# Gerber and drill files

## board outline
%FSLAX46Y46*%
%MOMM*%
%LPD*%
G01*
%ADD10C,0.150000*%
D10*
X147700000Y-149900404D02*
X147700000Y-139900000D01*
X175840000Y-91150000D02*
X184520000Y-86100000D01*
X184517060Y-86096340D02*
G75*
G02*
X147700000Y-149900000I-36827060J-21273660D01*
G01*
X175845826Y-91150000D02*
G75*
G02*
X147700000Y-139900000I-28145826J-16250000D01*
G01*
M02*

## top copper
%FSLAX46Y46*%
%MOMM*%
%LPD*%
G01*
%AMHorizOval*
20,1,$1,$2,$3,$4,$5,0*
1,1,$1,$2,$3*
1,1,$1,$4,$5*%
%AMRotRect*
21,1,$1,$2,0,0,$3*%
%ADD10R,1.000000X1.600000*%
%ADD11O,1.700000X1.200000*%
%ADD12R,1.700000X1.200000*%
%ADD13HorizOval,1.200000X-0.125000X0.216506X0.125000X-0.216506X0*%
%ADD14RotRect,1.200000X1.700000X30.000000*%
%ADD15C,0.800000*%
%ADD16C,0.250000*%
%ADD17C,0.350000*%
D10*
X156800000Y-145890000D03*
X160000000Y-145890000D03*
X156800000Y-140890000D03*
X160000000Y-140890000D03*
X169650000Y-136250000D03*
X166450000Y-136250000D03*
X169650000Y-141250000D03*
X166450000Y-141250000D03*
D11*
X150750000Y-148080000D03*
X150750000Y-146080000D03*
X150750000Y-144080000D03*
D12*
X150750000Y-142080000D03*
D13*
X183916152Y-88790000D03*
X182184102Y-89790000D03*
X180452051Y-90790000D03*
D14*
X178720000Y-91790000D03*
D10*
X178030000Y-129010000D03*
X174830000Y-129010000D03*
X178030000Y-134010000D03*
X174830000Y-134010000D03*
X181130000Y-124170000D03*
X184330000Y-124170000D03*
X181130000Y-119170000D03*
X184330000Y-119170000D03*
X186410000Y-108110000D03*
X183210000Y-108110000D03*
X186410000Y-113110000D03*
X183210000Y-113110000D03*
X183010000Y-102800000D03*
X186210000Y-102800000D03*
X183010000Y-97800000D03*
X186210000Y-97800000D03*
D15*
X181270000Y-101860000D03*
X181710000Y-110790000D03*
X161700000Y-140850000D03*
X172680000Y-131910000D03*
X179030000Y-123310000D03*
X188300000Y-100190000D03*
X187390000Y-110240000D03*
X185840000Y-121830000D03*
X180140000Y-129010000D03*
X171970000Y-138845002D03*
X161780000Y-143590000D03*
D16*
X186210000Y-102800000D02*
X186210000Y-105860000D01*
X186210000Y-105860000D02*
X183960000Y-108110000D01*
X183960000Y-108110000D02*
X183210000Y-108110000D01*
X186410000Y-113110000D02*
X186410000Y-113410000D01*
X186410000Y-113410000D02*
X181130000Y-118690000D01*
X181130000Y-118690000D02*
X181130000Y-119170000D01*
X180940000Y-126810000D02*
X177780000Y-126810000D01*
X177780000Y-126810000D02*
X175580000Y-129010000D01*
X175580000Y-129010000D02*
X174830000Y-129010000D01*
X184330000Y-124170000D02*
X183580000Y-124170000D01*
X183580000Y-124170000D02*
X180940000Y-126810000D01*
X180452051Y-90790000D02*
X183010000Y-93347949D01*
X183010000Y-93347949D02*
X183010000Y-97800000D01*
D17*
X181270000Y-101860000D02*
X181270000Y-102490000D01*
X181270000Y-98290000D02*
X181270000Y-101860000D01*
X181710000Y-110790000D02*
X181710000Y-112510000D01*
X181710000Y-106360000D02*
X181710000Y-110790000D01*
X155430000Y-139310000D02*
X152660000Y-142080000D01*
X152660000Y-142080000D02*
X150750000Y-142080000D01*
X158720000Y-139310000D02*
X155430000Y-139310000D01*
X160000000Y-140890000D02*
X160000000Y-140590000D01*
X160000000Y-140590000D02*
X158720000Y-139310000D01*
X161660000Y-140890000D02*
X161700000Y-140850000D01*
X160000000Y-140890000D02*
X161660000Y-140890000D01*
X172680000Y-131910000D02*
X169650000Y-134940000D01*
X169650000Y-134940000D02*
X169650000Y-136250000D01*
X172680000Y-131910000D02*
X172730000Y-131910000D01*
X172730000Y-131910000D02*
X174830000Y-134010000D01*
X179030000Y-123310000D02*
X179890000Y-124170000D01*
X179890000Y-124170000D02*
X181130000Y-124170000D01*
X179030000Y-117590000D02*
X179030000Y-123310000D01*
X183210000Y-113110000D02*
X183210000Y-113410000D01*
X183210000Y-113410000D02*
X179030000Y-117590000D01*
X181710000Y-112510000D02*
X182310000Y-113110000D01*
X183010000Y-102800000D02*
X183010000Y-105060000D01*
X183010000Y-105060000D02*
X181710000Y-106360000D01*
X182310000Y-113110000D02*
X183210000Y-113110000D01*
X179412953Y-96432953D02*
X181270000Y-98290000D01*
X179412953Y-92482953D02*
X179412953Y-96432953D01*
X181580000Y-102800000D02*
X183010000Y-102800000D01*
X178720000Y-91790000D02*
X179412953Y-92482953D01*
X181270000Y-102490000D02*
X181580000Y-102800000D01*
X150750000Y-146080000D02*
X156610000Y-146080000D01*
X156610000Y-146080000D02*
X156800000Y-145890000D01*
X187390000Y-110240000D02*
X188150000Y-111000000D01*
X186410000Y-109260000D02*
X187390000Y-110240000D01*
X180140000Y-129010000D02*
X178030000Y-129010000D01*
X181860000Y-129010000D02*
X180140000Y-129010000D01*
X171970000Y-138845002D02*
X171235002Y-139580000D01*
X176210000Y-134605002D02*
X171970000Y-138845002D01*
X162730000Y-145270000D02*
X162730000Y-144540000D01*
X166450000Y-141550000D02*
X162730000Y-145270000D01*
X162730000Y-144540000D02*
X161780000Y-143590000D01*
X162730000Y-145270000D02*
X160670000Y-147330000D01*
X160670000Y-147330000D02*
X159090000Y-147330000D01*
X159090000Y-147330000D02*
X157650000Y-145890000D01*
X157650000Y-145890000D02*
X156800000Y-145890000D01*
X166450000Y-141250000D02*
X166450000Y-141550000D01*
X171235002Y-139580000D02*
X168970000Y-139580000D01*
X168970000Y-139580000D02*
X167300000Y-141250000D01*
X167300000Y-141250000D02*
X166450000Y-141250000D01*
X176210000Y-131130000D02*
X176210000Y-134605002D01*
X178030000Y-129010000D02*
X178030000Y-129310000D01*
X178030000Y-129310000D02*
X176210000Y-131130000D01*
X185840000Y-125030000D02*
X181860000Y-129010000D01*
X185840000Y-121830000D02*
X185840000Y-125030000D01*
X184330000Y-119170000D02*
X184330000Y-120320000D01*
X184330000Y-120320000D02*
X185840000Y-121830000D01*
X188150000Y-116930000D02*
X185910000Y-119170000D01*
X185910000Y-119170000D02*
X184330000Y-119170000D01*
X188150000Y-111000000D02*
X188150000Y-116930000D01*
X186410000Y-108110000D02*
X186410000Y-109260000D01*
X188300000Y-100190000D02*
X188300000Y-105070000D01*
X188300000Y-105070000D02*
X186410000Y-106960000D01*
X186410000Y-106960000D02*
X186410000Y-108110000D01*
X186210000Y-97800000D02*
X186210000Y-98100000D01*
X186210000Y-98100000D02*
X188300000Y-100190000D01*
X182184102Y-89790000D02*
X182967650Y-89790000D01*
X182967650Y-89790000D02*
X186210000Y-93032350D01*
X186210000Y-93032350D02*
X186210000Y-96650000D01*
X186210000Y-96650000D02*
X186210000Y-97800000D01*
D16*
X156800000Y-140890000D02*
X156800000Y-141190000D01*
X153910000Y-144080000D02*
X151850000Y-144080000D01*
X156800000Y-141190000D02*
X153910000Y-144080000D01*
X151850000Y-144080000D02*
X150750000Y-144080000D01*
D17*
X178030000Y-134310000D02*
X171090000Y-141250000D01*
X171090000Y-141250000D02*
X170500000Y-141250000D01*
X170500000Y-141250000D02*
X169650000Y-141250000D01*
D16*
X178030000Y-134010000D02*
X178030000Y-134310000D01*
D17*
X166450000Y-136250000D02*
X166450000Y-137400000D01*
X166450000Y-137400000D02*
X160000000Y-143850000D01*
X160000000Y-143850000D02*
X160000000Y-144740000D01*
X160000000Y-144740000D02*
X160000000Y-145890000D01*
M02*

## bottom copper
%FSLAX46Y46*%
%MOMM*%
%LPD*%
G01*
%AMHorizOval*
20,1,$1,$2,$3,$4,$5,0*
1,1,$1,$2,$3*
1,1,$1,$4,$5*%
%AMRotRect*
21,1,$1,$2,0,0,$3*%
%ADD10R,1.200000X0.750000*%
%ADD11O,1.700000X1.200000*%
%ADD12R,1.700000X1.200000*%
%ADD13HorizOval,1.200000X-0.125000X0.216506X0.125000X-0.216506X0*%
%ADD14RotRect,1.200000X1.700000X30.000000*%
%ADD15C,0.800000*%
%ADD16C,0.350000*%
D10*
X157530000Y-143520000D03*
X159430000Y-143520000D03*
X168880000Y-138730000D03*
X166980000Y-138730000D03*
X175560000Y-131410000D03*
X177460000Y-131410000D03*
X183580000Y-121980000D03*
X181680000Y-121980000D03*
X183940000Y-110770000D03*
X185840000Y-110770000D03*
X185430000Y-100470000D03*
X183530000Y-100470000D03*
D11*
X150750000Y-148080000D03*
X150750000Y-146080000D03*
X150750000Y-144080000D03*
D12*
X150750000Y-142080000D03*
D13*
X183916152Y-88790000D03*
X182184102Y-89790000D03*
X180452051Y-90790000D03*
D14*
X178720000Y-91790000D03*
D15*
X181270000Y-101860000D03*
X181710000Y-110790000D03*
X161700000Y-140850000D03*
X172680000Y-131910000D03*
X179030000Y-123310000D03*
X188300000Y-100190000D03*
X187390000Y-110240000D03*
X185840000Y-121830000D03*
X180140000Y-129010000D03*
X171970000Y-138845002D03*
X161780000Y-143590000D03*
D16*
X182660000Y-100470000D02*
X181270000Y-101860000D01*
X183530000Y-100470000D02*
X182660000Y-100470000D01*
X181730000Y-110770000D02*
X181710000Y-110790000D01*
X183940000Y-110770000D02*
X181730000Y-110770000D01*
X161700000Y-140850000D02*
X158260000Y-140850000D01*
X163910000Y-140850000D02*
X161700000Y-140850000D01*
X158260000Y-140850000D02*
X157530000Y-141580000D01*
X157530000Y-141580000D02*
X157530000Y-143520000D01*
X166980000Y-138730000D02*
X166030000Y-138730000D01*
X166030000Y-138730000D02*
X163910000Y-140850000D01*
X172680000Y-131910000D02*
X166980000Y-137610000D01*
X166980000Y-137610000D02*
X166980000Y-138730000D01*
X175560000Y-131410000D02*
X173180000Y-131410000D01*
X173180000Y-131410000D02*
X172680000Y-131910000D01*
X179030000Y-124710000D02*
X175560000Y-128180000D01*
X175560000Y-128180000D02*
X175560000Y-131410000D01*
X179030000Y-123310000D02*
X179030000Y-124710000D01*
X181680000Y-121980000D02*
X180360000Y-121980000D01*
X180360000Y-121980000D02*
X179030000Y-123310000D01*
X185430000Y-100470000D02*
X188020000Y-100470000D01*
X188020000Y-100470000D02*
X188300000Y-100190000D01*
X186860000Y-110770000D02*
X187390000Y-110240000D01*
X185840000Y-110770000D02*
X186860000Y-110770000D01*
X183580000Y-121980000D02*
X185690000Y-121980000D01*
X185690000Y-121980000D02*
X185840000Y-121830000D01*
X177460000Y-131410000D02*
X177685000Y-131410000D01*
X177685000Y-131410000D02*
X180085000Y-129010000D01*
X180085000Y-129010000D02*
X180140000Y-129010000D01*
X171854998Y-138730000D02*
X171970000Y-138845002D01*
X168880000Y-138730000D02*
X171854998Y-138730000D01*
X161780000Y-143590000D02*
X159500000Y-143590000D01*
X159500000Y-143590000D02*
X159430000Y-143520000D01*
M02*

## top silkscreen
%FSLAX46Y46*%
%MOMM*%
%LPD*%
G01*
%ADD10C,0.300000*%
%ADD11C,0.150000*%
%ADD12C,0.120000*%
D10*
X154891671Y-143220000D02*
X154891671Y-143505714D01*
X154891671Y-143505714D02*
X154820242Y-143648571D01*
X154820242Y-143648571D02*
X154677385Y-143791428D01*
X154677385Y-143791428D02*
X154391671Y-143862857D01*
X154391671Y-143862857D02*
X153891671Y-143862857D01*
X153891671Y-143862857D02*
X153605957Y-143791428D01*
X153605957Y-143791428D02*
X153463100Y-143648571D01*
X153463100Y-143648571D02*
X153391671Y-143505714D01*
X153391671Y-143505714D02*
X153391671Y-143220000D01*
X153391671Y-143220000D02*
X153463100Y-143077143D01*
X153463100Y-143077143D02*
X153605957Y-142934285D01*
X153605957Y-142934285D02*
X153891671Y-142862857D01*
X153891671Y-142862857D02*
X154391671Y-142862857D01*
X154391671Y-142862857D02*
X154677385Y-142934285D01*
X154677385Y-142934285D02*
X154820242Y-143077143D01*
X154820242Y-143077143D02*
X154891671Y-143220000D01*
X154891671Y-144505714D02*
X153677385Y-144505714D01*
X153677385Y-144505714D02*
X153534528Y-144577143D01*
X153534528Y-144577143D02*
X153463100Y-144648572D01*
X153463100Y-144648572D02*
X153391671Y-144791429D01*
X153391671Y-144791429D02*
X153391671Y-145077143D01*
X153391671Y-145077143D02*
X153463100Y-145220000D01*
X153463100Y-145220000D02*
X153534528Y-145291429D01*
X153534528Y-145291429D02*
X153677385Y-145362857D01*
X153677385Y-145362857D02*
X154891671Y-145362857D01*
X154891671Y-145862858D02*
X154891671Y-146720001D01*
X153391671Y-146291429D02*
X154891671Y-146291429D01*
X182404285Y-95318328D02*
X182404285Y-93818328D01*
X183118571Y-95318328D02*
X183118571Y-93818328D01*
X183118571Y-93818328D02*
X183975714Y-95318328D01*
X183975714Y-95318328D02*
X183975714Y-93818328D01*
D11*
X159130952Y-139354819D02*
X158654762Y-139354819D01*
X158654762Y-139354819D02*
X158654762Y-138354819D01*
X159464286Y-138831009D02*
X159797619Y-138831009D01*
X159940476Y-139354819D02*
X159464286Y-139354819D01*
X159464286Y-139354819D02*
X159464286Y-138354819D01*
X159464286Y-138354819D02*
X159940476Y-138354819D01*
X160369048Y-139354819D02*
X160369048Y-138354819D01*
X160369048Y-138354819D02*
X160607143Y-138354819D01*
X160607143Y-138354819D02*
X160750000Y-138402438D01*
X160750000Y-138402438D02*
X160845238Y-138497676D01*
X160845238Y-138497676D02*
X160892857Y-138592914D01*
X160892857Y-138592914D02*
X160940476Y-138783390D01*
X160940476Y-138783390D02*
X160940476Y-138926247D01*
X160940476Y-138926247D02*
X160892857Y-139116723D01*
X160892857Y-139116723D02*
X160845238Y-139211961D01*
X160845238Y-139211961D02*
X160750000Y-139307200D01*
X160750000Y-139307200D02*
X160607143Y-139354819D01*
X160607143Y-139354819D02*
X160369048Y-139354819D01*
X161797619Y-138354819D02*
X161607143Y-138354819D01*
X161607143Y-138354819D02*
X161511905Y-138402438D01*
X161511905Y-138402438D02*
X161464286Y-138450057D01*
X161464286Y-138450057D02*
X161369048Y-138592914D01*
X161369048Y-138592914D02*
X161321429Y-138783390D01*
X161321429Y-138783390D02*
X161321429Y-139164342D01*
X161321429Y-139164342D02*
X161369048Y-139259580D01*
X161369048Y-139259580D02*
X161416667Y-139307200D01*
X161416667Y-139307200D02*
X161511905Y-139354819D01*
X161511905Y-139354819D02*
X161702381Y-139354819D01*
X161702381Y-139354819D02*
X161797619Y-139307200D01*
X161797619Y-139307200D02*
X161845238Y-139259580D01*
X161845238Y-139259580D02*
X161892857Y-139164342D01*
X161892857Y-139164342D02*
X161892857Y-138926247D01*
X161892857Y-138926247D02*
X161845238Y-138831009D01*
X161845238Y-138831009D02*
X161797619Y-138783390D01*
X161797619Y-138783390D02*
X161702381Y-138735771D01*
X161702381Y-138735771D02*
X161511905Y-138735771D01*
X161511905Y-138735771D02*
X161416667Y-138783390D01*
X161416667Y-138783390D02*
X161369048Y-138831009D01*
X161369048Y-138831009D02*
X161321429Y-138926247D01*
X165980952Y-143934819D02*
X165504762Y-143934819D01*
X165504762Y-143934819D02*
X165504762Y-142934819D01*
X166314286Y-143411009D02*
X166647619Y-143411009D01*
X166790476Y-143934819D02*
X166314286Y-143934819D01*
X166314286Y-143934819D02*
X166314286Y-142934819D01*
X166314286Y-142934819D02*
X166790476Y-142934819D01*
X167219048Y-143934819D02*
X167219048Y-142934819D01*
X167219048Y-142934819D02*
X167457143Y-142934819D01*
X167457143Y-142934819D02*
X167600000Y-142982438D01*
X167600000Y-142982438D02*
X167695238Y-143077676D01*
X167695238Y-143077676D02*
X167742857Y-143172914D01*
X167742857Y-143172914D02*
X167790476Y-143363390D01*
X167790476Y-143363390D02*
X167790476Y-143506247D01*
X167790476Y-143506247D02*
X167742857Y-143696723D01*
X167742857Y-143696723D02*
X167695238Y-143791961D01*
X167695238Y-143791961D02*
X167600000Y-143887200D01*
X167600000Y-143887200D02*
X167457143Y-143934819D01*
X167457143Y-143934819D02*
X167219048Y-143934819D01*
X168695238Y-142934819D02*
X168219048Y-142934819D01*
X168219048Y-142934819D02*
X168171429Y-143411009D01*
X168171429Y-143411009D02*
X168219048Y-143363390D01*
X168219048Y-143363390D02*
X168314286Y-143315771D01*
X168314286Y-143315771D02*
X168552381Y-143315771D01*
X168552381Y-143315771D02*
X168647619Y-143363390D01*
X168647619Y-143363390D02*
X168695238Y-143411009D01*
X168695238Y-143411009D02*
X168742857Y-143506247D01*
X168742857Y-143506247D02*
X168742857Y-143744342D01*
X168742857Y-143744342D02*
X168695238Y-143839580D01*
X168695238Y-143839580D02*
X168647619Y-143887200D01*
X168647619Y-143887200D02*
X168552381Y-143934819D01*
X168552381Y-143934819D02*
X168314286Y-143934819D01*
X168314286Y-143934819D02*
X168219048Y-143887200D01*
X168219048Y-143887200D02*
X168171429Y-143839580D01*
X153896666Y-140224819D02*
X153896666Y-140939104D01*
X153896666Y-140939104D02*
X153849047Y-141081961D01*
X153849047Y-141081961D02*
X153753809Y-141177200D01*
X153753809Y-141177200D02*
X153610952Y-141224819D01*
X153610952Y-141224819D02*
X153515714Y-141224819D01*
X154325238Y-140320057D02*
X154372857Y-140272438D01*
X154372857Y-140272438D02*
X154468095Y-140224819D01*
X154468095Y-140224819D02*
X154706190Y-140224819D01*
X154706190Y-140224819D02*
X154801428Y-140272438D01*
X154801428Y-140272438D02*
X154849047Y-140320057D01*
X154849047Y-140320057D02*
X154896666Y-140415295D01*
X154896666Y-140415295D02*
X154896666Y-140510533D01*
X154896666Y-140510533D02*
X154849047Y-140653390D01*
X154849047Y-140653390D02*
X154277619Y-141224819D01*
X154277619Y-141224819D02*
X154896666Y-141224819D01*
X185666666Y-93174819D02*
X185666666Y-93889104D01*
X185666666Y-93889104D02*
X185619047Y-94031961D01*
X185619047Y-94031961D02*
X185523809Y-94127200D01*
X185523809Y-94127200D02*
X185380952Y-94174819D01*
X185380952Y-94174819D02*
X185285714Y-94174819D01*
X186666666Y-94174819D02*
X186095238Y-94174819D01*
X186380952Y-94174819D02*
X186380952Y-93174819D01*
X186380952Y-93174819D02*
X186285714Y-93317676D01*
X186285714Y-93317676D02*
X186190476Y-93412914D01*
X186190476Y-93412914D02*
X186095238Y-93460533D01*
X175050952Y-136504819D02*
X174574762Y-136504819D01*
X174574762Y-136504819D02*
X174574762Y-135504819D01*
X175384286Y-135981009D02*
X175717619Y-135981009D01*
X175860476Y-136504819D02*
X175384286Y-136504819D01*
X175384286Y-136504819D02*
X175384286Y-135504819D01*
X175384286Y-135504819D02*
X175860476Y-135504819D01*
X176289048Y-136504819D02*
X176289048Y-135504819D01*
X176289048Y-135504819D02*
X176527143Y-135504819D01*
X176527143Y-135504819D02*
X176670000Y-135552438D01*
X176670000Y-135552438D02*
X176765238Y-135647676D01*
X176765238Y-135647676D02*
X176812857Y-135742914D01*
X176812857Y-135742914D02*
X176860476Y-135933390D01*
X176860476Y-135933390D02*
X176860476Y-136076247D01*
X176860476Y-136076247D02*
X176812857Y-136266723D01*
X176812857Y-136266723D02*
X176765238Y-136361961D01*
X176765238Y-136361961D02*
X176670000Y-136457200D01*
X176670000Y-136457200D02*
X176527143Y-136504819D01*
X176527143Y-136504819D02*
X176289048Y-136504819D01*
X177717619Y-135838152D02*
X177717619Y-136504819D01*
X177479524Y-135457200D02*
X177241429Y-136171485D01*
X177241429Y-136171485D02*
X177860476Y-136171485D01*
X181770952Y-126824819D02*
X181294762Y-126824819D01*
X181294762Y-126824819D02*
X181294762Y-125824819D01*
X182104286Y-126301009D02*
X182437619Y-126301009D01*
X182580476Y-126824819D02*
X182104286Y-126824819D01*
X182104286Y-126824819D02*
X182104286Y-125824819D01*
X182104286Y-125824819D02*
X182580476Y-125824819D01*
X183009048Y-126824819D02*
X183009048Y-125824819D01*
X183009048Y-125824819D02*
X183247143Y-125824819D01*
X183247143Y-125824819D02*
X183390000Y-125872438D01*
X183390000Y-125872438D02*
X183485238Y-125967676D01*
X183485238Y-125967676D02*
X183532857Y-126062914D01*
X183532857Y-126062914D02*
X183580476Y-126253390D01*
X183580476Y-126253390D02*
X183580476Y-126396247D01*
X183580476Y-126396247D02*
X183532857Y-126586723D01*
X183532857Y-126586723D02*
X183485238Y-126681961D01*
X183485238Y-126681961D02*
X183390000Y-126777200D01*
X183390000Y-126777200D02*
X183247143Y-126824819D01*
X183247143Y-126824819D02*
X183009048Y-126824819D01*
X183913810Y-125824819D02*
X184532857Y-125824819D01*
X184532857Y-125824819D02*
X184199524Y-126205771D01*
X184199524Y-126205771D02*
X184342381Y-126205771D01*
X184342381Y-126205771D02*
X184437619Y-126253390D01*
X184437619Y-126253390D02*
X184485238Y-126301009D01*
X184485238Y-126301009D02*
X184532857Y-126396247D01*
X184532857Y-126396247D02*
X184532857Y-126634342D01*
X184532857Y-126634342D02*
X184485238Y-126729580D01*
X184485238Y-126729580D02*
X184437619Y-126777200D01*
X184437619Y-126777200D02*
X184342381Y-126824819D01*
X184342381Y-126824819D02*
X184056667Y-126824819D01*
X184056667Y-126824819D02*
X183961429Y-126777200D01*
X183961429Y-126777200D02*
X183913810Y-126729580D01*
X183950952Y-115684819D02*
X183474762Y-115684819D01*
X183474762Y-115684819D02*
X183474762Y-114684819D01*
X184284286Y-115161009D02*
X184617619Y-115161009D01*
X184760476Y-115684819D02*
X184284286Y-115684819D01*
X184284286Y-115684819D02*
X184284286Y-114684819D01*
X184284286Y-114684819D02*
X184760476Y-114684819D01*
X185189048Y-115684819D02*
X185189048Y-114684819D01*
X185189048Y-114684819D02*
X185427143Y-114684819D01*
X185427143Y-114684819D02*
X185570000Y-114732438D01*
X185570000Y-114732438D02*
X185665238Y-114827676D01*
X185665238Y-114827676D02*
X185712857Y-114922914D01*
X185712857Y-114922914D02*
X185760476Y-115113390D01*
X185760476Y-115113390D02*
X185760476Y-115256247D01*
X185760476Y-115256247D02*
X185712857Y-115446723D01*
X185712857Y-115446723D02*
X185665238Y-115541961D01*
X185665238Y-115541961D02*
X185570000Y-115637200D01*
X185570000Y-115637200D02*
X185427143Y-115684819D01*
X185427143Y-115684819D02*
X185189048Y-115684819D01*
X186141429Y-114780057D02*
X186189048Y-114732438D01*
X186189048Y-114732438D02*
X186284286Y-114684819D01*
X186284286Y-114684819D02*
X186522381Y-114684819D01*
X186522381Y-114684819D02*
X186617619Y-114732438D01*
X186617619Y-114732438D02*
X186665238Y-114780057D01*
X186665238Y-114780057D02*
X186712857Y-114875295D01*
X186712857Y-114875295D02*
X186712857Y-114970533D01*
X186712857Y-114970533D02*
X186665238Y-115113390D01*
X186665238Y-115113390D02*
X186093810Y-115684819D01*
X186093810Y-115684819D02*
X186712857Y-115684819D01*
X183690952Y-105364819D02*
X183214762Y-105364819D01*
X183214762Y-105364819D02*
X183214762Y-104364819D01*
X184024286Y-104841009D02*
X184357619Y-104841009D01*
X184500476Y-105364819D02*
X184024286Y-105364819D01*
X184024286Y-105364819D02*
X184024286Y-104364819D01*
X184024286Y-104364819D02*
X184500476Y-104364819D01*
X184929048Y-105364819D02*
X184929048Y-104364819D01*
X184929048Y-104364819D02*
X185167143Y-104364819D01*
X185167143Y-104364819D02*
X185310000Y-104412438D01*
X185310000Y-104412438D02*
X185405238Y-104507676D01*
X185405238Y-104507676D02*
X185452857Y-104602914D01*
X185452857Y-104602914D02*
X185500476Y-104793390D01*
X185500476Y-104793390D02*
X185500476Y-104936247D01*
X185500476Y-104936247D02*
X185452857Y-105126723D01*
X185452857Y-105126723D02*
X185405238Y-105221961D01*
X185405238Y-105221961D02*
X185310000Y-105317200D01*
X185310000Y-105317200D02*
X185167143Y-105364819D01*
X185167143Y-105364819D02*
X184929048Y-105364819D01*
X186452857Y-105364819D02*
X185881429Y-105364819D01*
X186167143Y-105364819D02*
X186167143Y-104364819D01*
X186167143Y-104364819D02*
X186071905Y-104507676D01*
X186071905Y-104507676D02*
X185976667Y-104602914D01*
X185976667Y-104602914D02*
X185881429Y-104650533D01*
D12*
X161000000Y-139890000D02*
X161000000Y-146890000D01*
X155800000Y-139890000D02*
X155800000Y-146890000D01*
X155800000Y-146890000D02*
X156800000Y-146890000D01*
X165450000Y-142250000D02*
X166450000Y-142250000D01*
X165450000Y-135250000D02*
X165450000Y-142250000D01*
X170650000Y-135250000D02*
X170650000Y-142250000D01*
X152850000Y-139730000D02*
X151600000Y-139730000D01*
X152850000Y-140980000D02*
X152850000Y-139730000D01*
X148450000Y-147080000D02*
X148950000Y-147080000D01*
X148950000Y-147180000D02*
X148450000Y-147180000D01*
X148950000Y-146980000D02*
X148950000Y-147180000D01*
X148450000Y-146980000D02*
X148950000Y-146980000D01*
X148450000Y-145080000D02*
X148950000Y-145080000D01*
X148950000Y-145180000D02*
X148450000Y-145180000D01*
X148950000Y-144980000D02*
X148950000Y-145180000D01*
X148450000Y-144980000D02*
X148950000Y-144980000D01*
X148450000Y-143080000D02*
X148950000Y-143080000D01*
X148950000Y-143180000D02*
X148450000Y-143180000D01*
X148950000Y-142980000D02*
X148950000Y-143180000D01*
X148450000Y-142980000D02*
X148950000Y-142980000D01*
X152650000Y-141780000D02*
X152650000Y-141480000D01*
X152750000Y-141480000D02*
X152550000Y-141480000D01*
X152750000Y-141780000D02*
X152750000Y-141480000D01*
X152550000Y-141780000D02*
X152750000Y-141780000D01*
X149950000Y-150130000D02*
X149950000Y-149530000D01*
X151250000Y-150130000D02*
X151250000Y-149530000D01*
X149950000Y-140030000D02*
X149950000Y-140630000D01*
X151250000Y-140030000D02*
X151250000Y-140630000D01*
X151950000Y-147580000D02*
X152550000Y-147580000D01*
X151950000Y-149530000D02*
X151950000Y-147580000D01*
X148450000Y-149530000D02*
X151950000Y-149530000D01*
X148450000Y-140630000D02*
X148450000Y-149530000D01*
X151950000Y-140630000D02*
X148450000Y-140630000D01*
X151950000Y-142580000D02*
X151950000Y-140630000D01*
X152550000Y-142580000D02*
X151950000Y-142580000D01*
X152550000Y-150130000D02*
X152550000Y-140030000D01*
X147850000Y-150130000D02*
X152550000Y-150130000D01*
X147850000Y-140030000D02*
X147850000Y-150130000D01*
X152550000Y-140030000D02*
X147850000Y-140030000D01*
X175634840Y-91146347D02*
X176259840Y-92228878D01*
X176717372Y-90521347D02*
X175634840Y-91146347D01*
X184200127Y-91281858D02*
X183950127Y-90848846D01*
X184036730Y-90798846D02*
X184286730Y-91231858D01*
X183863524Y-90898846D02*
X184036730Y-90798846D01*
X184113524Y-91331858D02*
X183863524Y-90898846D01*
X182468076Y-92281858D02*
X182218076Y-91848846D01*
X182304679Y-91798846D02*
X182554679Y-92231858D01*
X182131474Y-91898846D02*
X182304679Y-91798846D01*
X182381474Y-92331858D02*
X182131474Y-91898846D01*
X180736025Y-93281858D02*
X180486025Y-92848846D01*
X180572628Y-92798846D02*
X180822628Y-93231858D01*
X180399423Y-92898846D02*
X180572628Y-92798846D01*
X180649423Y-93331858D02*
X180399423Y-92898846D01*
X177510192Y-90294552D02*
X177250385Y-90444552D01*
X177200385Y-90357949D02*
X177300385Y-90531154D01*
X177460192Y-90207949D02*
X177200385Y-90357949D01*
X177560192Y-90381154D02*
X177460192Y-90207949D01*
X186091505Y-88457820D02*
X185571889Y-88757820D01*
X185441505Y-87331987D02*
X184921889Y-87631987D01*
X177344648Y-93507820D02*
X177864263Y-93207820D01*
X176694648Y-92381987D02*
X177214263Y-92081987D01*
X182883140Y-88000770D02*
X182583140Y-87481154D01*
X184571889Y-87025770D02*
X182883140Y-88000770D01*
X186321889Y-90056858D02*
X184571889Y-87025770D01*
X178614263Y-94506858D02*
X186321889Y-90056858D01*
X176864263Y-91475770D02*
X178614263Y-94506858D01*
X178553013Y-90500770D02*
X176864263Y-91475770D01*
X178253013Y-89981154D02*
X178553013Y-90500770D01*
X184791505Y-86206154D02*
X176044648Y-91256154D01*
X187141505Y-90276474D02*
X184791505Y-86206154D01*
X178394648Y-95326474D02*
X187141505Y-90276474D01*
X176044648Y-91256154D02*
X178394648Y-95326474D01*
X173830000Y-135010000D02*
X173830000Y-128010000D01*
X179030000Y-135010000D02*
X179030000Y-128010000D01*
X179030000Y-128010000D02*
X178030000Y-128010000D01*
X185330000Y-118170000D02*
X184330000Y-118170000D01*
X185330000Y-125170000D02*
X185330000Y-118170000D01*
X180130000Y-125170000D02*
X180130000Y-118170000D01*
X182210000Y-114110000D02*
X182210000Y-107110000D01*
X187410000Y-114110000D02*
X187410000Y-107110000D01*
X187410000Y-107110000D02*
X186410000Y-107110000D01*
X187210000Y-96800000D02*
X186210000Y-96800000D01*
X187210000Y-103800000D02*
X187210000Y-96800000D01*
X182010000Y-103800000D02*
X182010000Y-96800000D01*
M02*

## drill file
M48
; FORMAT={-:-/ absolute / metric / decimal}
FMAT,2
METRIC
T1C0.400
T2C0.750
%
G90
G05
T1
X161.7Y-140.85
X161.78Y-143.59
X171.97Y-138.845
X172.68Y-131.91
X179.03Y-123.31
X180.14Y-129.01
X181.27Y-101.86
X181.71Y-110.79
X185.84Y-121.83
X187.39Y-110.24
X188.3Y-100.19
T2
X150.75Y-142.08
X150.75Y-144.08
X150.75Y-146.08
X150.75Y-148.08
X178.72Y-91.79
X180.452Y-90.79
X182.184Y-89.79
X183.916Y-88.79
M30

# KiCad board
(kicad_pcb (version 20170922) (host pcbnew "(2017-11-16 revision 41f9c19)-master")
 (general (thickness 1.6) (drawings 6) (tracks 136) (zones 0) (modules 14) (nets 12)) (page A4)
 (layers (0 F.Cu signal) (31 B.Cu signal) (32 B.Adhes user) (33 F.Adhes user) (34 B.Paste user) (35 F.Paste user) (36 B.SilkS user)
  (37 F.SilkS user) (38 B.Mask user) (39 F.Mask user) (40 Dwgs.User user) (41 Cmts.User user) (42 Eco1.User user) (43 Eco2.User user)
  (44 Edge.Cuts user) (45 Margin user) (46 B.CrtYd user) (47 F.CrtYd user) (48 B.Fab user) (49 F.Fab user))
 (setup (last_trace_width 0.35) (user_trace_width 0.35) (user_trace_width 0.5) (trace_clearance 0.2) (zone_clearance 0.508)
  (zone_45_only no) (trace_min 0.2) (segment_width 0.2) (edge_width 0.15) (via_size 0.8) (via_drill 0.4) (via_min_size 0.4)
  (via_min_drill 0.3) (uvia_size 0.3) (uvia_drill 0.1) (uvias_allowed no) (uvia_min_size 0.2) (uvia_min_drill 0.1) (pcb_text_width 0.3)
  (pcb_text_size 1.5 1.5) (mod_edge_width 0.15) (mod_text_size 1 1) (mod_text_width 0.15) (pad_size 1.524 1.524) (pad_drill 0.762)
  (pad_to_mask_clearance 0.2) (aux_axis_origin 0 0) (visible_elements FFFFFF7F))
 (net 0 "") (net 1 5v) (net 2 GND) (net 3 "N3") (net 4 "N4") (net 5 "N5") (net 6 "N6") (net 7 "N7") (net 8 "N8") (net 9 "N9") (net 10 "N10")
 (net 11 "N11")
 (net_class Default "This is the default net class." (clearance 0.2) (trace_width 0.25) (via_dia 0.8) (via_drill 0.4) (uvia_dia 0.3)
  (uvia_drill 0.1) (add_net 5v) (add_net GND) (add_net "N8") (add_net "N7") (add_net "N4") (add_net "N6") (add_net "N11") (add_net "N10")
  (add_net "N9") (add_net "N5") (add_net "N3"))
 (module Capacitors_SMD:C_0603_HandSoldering (layer B.Cu) (at 158.48 143.52)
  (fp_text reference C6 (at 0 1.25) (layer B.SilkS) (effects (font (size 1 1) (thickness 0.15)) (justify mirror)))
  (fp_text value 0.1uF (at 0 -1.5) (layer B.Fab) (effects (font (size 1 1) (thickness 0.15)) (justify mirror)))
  (pad 1 smd rect (at -0.95 0) (size 1.2 0.75) (layers B.Cu B.Paste B.Mask) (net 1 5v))
  (pad 2 smd rect (at 0.95 0) (size 1.2 0.75) (layers B.Cu B.Paste B.Mask) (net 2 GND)))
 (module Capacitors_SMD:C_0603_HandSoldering (layer B.Cu) (at 167.93 138.73)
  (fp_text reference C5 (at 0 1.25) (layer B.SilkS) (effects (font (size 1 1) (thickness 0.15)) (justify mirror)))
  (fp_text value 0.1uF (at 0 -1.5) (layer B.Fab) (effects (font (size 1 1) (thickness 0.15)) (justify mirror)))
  (pad 2 smd rect (at 0.95 0) (size 1.2 0.75) (layers B.Cu B.Paste B.Mask) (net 2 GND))
  (pad 1 smd rect (at -0.95 0) (size 1.2 0.75) (layers B.Cu B.Paste B.Mask) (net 1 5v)))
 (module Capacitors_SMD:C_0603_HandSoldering (layer B.Cu) (at 176.51 131.41)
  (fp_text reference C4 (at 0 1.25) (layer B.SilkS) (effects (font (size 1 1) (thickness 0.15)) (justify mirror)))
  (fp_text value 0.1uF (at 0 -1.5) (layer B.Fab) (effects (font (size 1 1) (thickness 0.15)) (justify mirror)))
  (pad 1 smd rect (at -0.95 0) (size 1.2 0.75) (layers B.Cu B.Paste B.Mask) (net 1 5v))
  (pad 2 smd rect (at 0.95 0) (size 1.2 0.75) (layers B.Cu B.Paste B.Mask) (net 2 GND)))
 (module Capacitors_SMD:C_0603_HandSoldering (layer B.Cu) (at 182.63 121.98)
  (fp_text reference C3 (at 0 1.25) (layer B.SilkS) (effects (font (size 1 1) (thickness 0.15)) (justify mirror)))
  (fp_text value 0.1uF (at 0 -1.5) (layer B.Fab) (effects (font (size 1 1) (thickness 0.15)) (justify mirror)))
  (pad 2 smd rect (at 0.95 0) (size 1.2 0.75) (layers B.Cu B.Paste B.Mask) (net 2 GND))
  (pad 1 smd rect (at -0.95 0) (size 1.2 0.75) (layers B.Cu B.Paste B.Mask) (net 1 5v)))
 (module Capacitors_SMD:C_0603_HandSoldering (layer B.Cu) (at 184.89 110.77)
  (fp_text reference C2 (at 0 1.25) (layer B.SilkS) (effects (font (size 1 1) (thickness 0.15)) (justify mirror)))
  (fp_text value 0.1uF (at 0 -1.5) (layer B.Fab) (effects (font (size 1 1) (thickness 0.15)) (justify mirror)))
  (pad 1 smd rect (at -0.95 0) (size 1.2 0.75) (layers B.Cu B.Paste B.Mask) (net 1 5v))
  (pad 2 smd rect (at 0.95 0) (size 1.2 0.75) (layers B.Cu B.Paste B.Mask) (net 2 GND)))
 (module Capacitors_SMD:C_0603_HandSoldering (layer B.Cu) (at 184.48 100.47)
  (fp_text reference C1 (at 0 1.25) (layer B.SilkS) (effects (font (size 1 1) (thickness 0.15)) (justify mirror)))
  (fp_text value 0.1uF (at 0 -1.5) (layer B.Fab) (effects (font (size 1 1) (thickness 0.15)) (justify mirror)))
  (pad 2 smd rect (at 0.95 0) (size 1.2 0.75) (layers B.Cu B.Paste B.Mask) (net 2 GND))
  (pad 1 smd rect (at -0.95 0) (size 1.2 0.75) (layers B.Cu B.Paste B.Mask) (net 1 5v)))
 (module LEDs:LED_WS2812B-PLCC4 (layer F.Cu) (at 158.4 143.39 270)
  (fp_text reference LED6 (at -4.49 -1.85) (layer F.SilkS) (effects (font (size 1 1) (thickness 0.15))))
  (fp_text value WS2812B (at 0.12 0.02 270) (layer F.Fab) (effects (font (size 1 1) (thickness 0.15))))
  (fp_line (start -3.5 -2.6) (end 3.5 -2.6) (layer F.SilkS) (width 0.12))
  (fp_line (start -3.5 2.6) (end 3.5 2.6) (layer F.SilkS) (width 0.12))
  (fp_line (start 3.5 2.6) (end 3.5 1.6) (layer F.SilkS) (width 0.12))
  (pad 3 smd rect (at 2.5 1.6 270) (size 1.6 1) (layers F.Cu F.Paste F.Mask) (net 2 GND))
  (pad 4 smd rect (at 2.5 -1.6 270) (size 1.6 1) (layers F.Cu F.Paste F.Mask) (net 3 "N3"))
  (pad 2 smd rect (at -2.5 1.6 270) (size 1.6 1) (layers F.Cu F.Paste F.Mask) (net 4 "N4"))
  (pad 1 smd rect (at -2.5 -1.6 270) (size 1.6 1) (layers F.Cu F.Paste F.Mask) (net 1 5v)))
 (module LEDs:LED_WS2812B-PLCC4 (layer F.Cu) (at 168.05 138.75 270)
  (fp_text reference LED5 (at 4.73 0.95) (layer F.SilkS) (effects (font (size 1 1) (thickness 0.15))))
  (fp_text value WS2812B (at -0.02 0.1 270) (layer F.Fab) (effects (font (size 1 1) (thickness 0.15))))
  (fp_line (start 3.5 2.6) (end 3.5 1.6) (layer F.SilkS) (width 0.12))
  (fp_line (start -3.5 2.6) (end 3.5 2.6) (layer F.SilkS) (width 0.12))
  (fp_line (start -3.5 -2.6) (end 3.5 -2.6) (layer F.SilkS) (width 0.12))
  (pad 1 smd rect (at -2.5 -1.6 270) (size 1.6 1) (layers F.Cu F.Paste F.Mask) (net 1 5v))
  (pad 2 smd rect (at -2.5 1.6 270) (size 1.6 1) (layers F.Cu F.Paste F.Mask) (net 3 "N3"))
  (pad 4 smd rect (at 2.5 -1.6 270) (size 1.6 1) (layers F.Cu F.Paste F.Mask) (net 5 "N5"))
  (pad 3 smd rect (at 2.5 1.6 270) (size 1.6 1) (layers F.Cu F.Paste F.Mask) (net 2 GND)))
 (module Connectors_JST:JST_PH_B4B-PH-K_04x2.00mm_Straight (layer F.Cu) (at 150.75 142.08 270)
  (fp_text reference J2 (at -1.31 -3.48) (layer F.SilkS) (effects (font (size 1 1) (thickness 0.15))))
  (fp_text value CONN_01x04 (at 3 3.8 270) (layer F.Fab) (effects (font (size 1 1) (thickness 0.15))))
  (fp_line (start -2.35 -2.1) (end -2.35 -0.85) (layer F.SilkS) (width 0.12))
  (fp_line (start -1.1 -2.1) (end -2.35 -2.1) (layer F.SilkS) (width 0.12))
  (fp_line (start 5 2.3) (end 5 1.8) (layer F.SilkS) (width 0.12))
  (fp_line (start 5.1 1.8) (end 5.1 2.3) (layer F.SilkS) (width 0.12))
  (fp_line (start 4.9 1.8) (end 5.1 1.8) (layer F.SilkS) (width 0.12))
  (fp_line (start 4.9 2.3) (end 4.9 1.8) (layer F.SilkS) (width 0.12))
  (fp_line (start 3 2.3) (end 3 1.8) (layer F.SilkS) (width 0.12))
  (fp_line (start 3.1 1.8) (end 3.1 2.3) (layer F.SilkS) (width 0.12))
  (fp_line (start 2.9 1.8) (end 3.1 1.8) (layer F.SilkS) (width 0.12))
  (fp_line (start 2.9 2.3) (end 2.9 1.8) (layer F.SilkS) (width 0.12))
  (fp_line (start 1 2.3) (end 1 1.8) (layer F.SilkS) (width 0.12))
  (fp_line (start 1.1 1.8) (end 1.1 2.3) (layer F.SilkS) (width 0.12))
  (fp_line (start 0.9 1.8) (end 1.1 1.8) (layer F.SilkS) (width 0.12))
  (fp_line (start 0.9 2.3) (end 0.9 1.8) (layer F.SilkS) (width 0.12))
  (fp_line (start -0.3 -1.9) (end -0.6 -1.9) (layer F.SilkS) (width 0.12))
  (fp_line (start -0.6 -2) (end -0.6 -1.8) (layer F.SilkS) (width 0.12))
  (fp_line (start -0.3 -2) (end -0.6 -2) (layer F.SilkS) (width 0.12))
  (fp_line (start -0.3 -1.8) (end -0.3 -2) (layer F.SilkS) (width 0.12))
  (fp_line (start 8.05 0.8) (end 7.45 0.8) (layer F.SilkS) (width 0.12))
  (fp_line (start 8.05 -0.5) (end 7.45 -0.5) (layer F.SilkS) (width 0.12))
  (fp_line (start -2.05 0.8) (end -1.45 0.8) (layer F.SilkS) (width 0.12))
  (fp_line (start -2.05 -0.5) (end -1.45 -0.5) (layer F.SilkS) (width 0.12))
  (fp_line (start 5.5 -1.2) (end 5.5 -1.8) (layer F.SilkS) (width 0.12))
  (fp_line (start 7.45 -1.2) (end 5.5 -1.2) (layer F.SilkS) (width 0.12))
  (fp_line (start 7.45 2.3) (end 7.45 -1.2) (layer F.SilkS) (width 0.12))
  (fp_line (start -1.45 2.3) (end 7.45 2.3) (layer F.SilkS) (width 0.12))
  (fp_line (start -1.45 -1.2) (end -1.45 2.3) (layer F.SilkS) (width 0.12))
  (fp_line (start 0.5 -1.2) (end -1.45 -1.2) (layer F.SilkS) (width 0.12))
  (fp_line (start 0.5 -1.8) (end 0.5 -1.2) (layer F.SilkS) (width 0.12))
  (fp_line (start 8.05 -1.8) (end -2.05 -1.8) (layer F.SilkS) (width 0.12))
  (fp_line (start 8.05 2.9) (end 8.05 -1.8) (layer F.SilkS) (width 0.12))
  (fp_line (start -2.05 2.9) (end 8.05 2.9) (layer F.SilkS) (width 0.12))
  (fp_line (start -2.05 -1.8) (end -2.05 2.9) (layer F.SilkS) (width 0.12))
  (pad 4 thru_hole oval (at 6 0 270) (size 1.2 1.7) (drill 0.75) (layers *.Cu *.Mask) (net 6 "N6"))
  (pad 3 thru_hole oval (at 4 0 270) (size 1.2 1.7) (drill 0.75) (layers *.Cu *.Mask) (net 2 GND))
  (pad 2 thru_hole oval (at 2 0 270) (size 1.2 1.7) (drill 0.75) (layers *.Cu *.Mask) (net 4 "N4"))
  (pad 1 thru_hole rect (at 0 0 270) (size 1.2 1.7) (drill 0.75) (layers *.Cu *.Mask) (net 1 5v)))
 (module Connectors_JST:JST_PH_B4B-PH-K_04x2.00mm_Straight (layer F.Cu) (at 178.72 91.79 30)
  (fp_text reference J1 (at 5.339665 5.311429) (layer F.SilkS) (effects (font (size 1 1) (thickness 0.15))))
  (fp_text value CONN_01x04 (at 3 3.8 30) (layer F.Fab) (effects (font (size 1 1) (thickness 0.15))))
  (fp_line (start -2.35 -2.1) (end -2.35 -0.85) (layer F.SilkS) (width 0.12))
  (fp_line (start -1.1 -2.1) (end -2.35 -2.1) (layer F.SilkS) (width 0.12))
  (fp_line (start 5 2.3) (end 5 1.8) (layer F.SilkS) (width 0.12))
  (fp_line (start 5.1 1.8) (end 5.1 2.3) (layer F.SilkS) (width 0.12))
  (fp_line (start 4.9 1.8) (end 5.1 1.8) (layer F.SilkS) (width 0.12))
  (fp_line (start 4.9 2.3) (end 4.9 1.8) (layer F.SilkS) (width 0.12))
  (fp_line (start 3 2.3) (end 3 1.8) (layer F.SilkS) (width 0.12))
  (fp_line (start 3.1 1.8) (end 3.1 2.3) (layer F.SilkS) (width 0.12))
  (fp_line (start 2.9 1.8) (end 3.1 1.8) (layer F.SilkS) (width 0.12))
  (fp_line (start 2.9 2.3) (end 2.9 1.8) (layer F.SilkS) (width 0.12))
  (fp_line (start 1 2.3) (end 1 1.8) (layer F.SilkS) (width 0.12))
  (fp_line (start 1.1 1.8) (end 1.1 2.3) (layer F.SilkS) (width 0.12))
  (fp_line (start 0.9 1.8) (end 1.1 1.8) (layer F.SilkS) (width 0.12))
  (fp_line (start 0.9 2.3) (end 0.9 1.8) (layer F.SilkS) (width 0.12))
  (fp_line (start -0.3 -1.9) (end -0.6 -1.9) (layer F.SilkS) (width 0.12))
  (fp_line (start -0.6 -2) (end -0.6 -1.8) (layer F.SilkS) (width 0.12))
  (fp_line (start -0.3 -2) (end -0.6 -2) (layer F.SilkS) (width 0.12))
  (fp_line (start -0.3 -1.8) (end -0.3 -2) (layer F.SilkS) (width 0.12))
  (fp_line (start 8.05 0.8) (end 7.45 0.8) (layer F.SilkS) (width 0.12))
  (fp_line (start 8.05 -0.5) (end 7.45 -0.5) (layer F.SilkS) (width 0.12))
  (fp_line (start -2.05 0.8) (end -1.45 0.8) (layer F.SilkS) (width 0.12))
  (fp_line (start -2.05 -0.5) (end -1.45 -0.5) (layer F.SilkS) (width 0.12))
  (fp_line (start 5.5 -1.2) (end 5.5 -1.8) (layer F.SilkS) (width 0.12))
  (fp_line (start 7.45 -1.2) (end 5.5 -1.2) (layer F.SilkS) (width 0.12))
  (fp_line (start 7.45 2.3) (end 7.45 -1.2) (layer F.SilkS) (width 0.12))
  (fp_line (start -1.45 2.3) (end 7.45 2.3) (layer F.SilkS) (width 0.12))
  (fp_line (start -1.45 -1.2) (end -1.45 2.3) (layer F.SilkS) (width 0.12))
  (fp_line (start 0.5 -1.2) (end -1.45 -1.2) (layer F.SilkS) (width 0.12))
  (fp_line (start 0.5 -1.8) (end 0.5 -1.2) (layer F.SilkS) (width 0.12))
  (fp_line (start 8.05 -1.8) (end -2.05 -1.8) (layer F.SilkS) (width 0.12))
  (fp_line (start 8.05 2.9) (end 8.05 -1.8) (layer F.SilkS) (width 0.12))
  (fp_line (start -2.05 2.9) (end 8.05 2.9) (layer F.SilkS) (width 0.12))
  (fp_line (start -2.05 -1.8) (end -2.05 2.9) (layer F.SilkS) (width 0.12))
  (pad 4 thru_hole oval (at 6 0 30) (size 1.2 1.7) (drill 0.75) (layers *.Cu *.Mask) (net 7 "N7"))
  (pad 3 thru_hole oval (at 4 0 30) (size 1.2 1.7) (drill 0.75) (layers *.Cu *.Mask) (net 2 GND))
  (pad 2 thru_hole oval (at 2 0 30) (size 1.2 1.7) (drill 0.75) (layers *.Cu *.Mask) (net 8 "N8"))
  (pad 1 thru_hole rect (at 0 0 30) (size 1.2 1.7) (drill 0.75) (layers *.Cu *.Mask) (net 1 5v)))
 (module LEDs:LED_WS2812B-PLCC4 (layer F.Cu) (at 176.43 131.51 90)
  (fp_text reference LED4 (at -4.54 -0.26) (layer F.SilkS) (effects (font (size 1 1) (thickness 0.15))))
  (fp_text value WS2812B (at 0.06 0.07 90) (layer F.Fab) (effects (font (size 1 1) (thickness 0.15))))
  (fp_line (start -3.5 -2.6) (end 3.5 -2.6) (layer F.SilkS) (width 0.12))
  (fp_line (start -3.5 2.6) (end 3.5 2.6) (layer F.SilkS) (width 0.12))
  (fp_line (start 3.5 2.6) (end 3.5 1.6) (layer F.SilkS) (width 0.12))
  (pad 3 smd rect (at 2.5 1.6 90) (size 1.6 1) (layers F.Cu F.Paste F.Mask) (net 2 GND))
  (pad 4 smd rect (at 2.5 -1.6 90) (size 1.6 1) (layers F.Cu F.Paste F.Mask) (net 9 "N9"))
  (pad 2 smd rect (at -2.5 1.6 90) (size 1.6 1) (layers F.Cu F.Paste F.Mask) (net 5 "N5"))
  (pad 1 smd rect (at -2.5 -1.6 90) (size 1.6 1) (layers F.Cu F.Paste F.Mask) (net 1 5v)))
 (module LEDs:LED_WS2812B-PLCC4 (layer F.Cu) (at 182.73 121.67 90)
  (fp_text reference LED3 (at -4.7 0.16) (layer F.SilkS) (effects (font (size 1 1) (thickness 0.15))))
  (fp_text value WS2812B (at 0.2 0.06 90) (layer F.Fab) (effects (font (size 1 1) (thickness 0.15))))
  (fp_line (start 3.5 2.6) (end 3.5 1.6) (layer F.SilkS) (width 0.12))
  (fp_line (start -3.5 2.6) (end 3.5 2.6) (layer F.SilkS) (width 0.12))
  (fp_line (start -3.5 -2.6) (end 3.5 -2.6) (layer F.SilkS) (width 0.12))
  (pad 1 smd rect (at -2.5 -1.6 90) (size 1.6 1) (layers F.Cu F.Paste F.Mask) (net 1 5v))
  (pad 2 smd rect (at -2.5 1.6 90) (size 1.6 1) (layers F.Cu F.Paste F.Mask) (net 9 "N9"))
  (pad 4 smd rect (at 2.5 -1.6 90) (size 1.6 1) (layers F.Cu F.Paste F.Mask) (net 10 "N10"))
  (pad 3 smd rect (at 2.5 1.6 90) (size 1.6 1) (layers F.Cu F.Paste F.Mask) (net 2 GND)))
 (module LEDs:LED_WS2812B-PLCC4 (layer F.Cu) (at 184.81 110.61 90)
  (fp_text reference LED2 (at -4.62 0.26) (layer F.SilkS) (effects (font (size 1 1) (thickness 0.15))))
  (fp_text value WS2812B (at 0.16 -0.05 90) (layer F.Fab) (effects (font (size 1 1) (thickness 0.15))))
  (fp_line (start -3.5 -2.6) (end 3.5 -2.6) (layer F.SilkS) (width 0.12))
  (fp_line (start -3.5 2.6) (end 3.5 2.6) (layer F.SilkS) (width 0.12))
  (fp_line (start 3.5 2.6) (end 3.5 1.6) (layer F.SilkS) (width 0.12))
  (pad 3 smd rect (at 2.5 1.6 90) (size 1.6 1) (layers F.Cu F.Paste F.Mask) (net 2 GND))
  (pad 4 smd rect (at 2.5 -1.6 90) (size 1.6 1) (layers F.Cu F.Paste F.Mask) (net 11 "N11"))
  (pad 2 smd rect (at -2.5 1.6 90) (size 1.6 1) (layers F.Cu F.Paste F.Mask) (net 10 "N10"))
  (pad 1 smd rect (at -2.5 -1.6 90) (size 1.6 1) (layers F.Cu F.Paste F.Mask) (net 1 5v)))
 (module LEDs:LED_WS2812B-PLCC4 (layer F.Cu) (at 184.61 100.3 90)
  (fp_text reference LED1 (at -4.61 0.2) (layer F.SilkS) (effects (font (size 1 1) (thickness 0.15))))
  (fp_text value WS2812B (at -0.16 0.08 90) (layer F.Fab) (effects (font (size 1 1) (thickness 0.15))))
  (fp_line (start 3.5 2.6) (end 3.5 1.6) (layer F.SilkS) (width 0.12))
  (fp_line (start -3.5 2.6) (end 3.5 2.6) (layer F.SilkS) (width 0.12))
  (fp_line (start -3.5 -2.6) (end 3.5 -2.6) (layer F.SilkS) (width 0.12))
  (pad 1 smd rect (at -2.5 -1.6 90) (size 1.6 1) (layers F.Cu F.Paste F.Mask) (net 1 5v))
  (pad 2 smd rect (at -2.5 1.6 90) (size 1.6 1) (layers F.Cu F.Paste F.Mask) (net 11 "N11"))
  (pad 4 smd rect (at 2.5 -1.6 90) (size 1.6 1) (layers F.Cu F.Paste F.Mask) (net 8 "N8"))
  (pad 3 smd rect (at 2.5 1.6 90) (size 1.6 1) (layers F.Cu F.Paste F.Mask) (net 2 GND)))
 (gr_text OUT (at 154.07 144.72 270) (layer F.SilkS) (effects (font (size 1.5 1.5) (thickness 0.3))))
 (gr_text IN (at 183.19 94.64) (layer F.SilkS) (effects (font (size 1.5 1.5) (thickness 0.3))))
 (gr_line (start 147.7 149.900404) (end 147.7 139.9) (layer Edge.Cuts) (width 0.15))
 (gr_line (start 175.84 91.15) (end 184.52 86.1) (layer Edge.Cuts) (width 0.15))
 (gr_arc (start 147.69 107.37) (end 147.7 149.9) (angle -120) (layer Edge.Cuts) (width 0.15))
 (gr_arc (start 147.7 107.4) (end 147.7 139.9) (angle -120) (layer Edge.Cuts) (width 0.15))
 (segment (start 186.21 102.8) (end 186.21 105.86) (width 0.25) (layer F.Cu) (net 11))
 (segment (start 186.21 105.86) (end 183.96 108.11) (width 0.25) (layer F.Cu) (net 11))
 (segment (start 183.96 108.11) (end 183.21 108.11) (width 0.25) (layer F.Cu) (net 11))
 (segment (start 186.41 113.11) (end 186.41 113.41) (width 0.25) (layer F.Cu) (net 10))
 (segment (start 186.41 113.41) (end 181.13 118.69) (width 0.25) (layer F.Cu) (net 10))
 (segment (start 181.13 118.69) (end 181.13 119.17) (width 0.25) (layer F.Cu) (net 10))
 (segment (start 180.94 126.81) (end 177.78 126.81) (width 0.25) (layer F.Cu) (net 9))
 (segment (start 177.78 126.81) (end 175.58 129.01) (width 0.25) (layer F.Cu) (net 9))
 (segment (start 175.58 129.01) (end 174.83 129.01) (width 0.25) (layer F.Cu) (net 9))
 (segment (start 184.33 124.17) (end 183.58 124.17) (width 0.25) (layer F.Cu) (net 9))
 (segment (start 183.58 124.17) (end 180.94 126.81) (width 0.25) (layer F.Cu) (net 9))
 (segment (start 180.452051 90.79) (end 183.01 93.347949) (width 0.25) (layer F.Cu) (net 8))
 (segment (start 183.01 93.347949) (end 183.01 97.8) (width 0.25) (layer F.Cu) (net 8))
 (segment (start 182.66 100.47) (end 181.27 101.86) (width 0.35) (layer B.Cu) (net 1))
 (segment (start 183.53 100.47) (end 182.66 100.47) (width 0.35) (layer B.Cu) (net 1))
 (segment (start 181.27 101.86) (end 181.27 102.49) (width 0.35) (layer F.Cu) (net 1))
 (segment (start 181.27 98.29) (end 181.27 101.86) (width 0.35) (layer F.Cu) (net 1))
 (via (at 181.27 101.86) (size 0.8) (drill 0.4) (layers F.Cu B.Cu) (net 1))
 (segment (start 181.73 110.77) (end 181.71 110.79) (width 0.35) (layer B.Cu) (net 1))
 (segment (start 183.94 110.77) (end 181.73 110.77) (width 0.35) (layer B.Cu) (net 1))
 (segment (start 181.71 110.79) (end 181.71 112.51) (width 0.35) (layer F.Cu) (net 1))
 (segment (start 181.71 106.36) (end 181.71 110.79) (width 0.35) (layer F.Cu) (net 1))
 (via (at 181.71 110.79) (size 0.8) (drill 0.4) (layers F.Cu B.Cu) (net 1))
 (segment (start 155.43 139.31) (end 152.66 142.08) (width 0.35) (layer F.Cu) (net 1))
 (segment (start 152.66 142.08) (end 150.75 142.08) (width 0.35) (layer F.Cu) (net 1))
 (segment (start 158.72 139.31) (end 155.43 139.31) (width 0.35) (layer F.Cu) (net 1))
 (segment (start 160 140.89) (end 160 140.59) (width 0.35) (layer F.Cu) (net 1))
 (segment (start 160 140.59) (end 158.72 139.31) (width 0.35) (layer F.Cu) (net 1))
 (segment (start 161.66 140.89) (end 161.7 140.85) (width 0.35) (layer F.Cu) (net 1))
 (segment (start 160 140.89) (end 161.66 140.89) (width 0.35) (layer F.Cu) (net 1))
 (segment (start 161.7 140.85) (end 158.26 140.85) (width 0.35) (layer B.Cu) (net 1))
 (segment (start 163.91 140.85) (end 161.7 140.85) (width 0.35) (layer B.Cu) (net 1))
 (via (at 161.7 140.85) (size 0.8) (drill 0.4) (layers F.Cu B.Cu) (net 1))
 (segment (start 158.26 140.85) (end 157.53 141.58) (width 0.35) (layer B.Cu) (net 1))
 (segment (start 157.53 141.58) (end 157.53 143.52) (width 0.35) (layer B.Cu) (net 1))
 (segment (start 166.98 138.73) (end 166.03 138.73) (width 0.35) (layer B.Cu) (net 1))
 (segment (start 166.03 138.73) (end 163.91 140.85) (width 0.35) (layer B.Cu) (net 1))
 (segment (start 172.68 131.91) (end 166.98 137.61) (width 0.35) (layer B.Cu) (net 1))
 (segment (start 166.98 137.61) (end 166.98 138.73) (width 0.35) (layer B.Cu) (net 1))
 (segment (start 172.68 131.91) (end 169.65 134.94) (width 0.35) (layer F.Cu) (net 1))
 (segment (start 169.65 134.94) (end 169.65 136.25) (width 0.35) (layer F.Cu) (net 1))
 (segment (start 172.68 131.91) (end 172.73 131.91) (width 0.35) (layer F.Cu) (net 1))
 (segment (start 172.73 131.91) (end 174.83 134.01) (width 0.35) (layer F.Cu) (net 1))
 (segment (start 175.56 131.41) (end 173.18 131.41) (width 0.35) (layer B.Cu) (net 1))
 (segment (start 173.18 131.41) (end 172.68 131.91) (width 0.35) (layer B.Cu) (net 1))
 (via (at 172.68 131.91) (size 0.8) (drill 0.4) (layers F.Cu B.Cu) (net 1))
 (segment (start 179.03 124.71) (end 175.56 128.18) (width 0.35) (layer B.Cu) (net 1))
 (segment (start 175.56 128.18) (end 175.56 131.41) (width 0.35) (layer B.Cu) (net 1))
 (segment (start 179.03 123.31) (end 179.03 124.71) (width 0.35) (layer B.Cu) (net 1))
 (segment (start 181.68 121.98) (end 180.36 121.98) (width 0.35) (layer B.Cu) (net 1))
 (segment (start 180.36 121.98) (end 179.03 123.31) (width 0.35) (layer B.Cu) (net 1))
 (via (at 179.03 123.31) (size 0.8) (drill 0.4) (layers F.Cu B.Cu) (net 1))
 (segment (start 179.03 123.31) (end 179.89 124.17) (width 0.35) (layer F.Cu) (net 1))
 (segment (start 179.89 124.17) (end 181.13 124.17) (width 0.35) (layer F.Cu) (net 1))
 (segment (start 179.03 117.59) (end 179.03 123.31) (width 0.35) (layer F.Cu) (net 1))
 (segment (start 183.21 113.11) (end 183.21 113.41) (width 0.35) (layer F.Cu) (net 1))
 (segment (start 183.21 113.41) (end 179.03 117.59) (width 0.35) (layer F.Cu) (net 1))
 (segment (start 181.71 112.51) (end 182.31 113.11) (width 0.35) (layer F.Cu) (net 1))
 (segment (start 183.01 102.8) (end 183.01 105.06) (width 0.35) (layer F.Cu) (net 1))
 (segment (start 183.01 105.06) (end 181.71 106.36) (width 0.35) (layer F.Cu) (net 1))
 (segment (start 182.31 113.11) (end 183.21 113.11) (width 0.35) (layer F.Cu) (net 1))
 (segment (start 179.412953 96.432953) (end 181.27 98.29) (width 0.35) (layer F.Cu) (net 1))
 (segment (start 179.412953 92.482953) (end 179.412953 96.432953) (width 0.35) (layer F.Cu) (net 1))
 (segment (start 181.58 102.8) (end 183.01 102.8) (width 0.35) (layer F.Cu) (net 1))
 (segment (start 178.72 91.79) (end 179.412953 92.482953) (width 0.35) (layer F.Cu) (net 1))
 (segment (start 181.27 102.49) (end 181.58 102.8) (width 0.35) (layer F.Cu) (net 1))
 (segment (start 150.75 146.08) (end 156.61 146.08) (width 0.35) (layer F.Cu) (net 2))
 (segment (start 156.61 146.08) (end 156.8 145.89) (width 0.35) (layer F.Cu) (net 2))
 (segment (start 185.43 100.47) (end 188.02 100.47) (width 0.35) (layer B.Cu) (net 2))
 (segment (start 188.02 100.47) (end 188.3 100.19) (width 0.35) (layer B.Cu) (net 2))
 (via (at 188.3 100.19) (size 0.8) (drill 0.4) (layers F.Cu B.Cu) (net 2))
 (segment (start 186.86 110.77) (end 187.39 110.24) (width 0.35) (layer B.Cu) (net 2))
 (segment (start 185.84 110.77) (end 186.86 110.77) (width 0.35) (layer B.Cu) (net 2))
 (segment (start 187.39 110.24) (end 188.15 111) (width 0.35) (layer F.Cu) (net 2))
 (via (at 187.39 110.24) (size 0.8) (drill 0.4) (layers F.Cu B.Cu) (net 2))
 (segment (start 186.41 109.26) (end 187.39 110.24) (width 0.35) (layer F.Cu) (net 2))
 (segment (start 183.58 121.98) (end 185.69 121.98) (width 0.35) (layer B.Cu) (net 2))
 (segment (start 185.69 121.98) (end 185.84 121.83) (width 0.35) (layer B.Cu) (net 2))
 (via (at 185.84 121.83) (size 0.8) (drill 0.4) (layers F.Cu B.Cu) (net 2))
 (segment (start 177.46 131.41) (end 177.685 131.41) (width 0.35) (layer B.Cu) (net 2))
 (segment (start 180.14 129.01) (end 178.03 129.01) (width 0.35) (layer F.Cu) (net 2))
 (segment (start 177.685 131.41) (end 180.085 129.01) (width 0.35) (layer B.Cu) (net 2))
 (segment (start 181.86 129.01) (end 180.14 129.01) (width 0.35) (layer F.Cu) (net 2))
 (via (at 180.14 129.01) (size 0.8) (drill 0.4) (layers F.Cu B.Cu) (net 2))
 (segment (start 180.085 129.01) (end 180.14 129.01) (width 0.35) (layer B.Cu) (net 2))
 (segment (start 171.854998 138.73) (end 171.97 138.845002) (width 0.35) (layer B.Cu) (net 2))
 (segment (start 171.97 138.845002) (end 171.235002 139.58) (width 0.35) (layer F.Cu) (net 2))
 (segment (start 168.88 138.73) (end 171.854998 138.73) (width 0.35) (layer B.Cu) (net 2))
 (segment (start 176.21 134.605002) (end 171.97 138.845002) (width 0.35) (layer F.Cu) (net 2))
 (via (at 171.97 138.845002) (size 0.8) (drill 0.4) (layers F.Cu B.Cu) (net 2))
 (segment (start 161.78 143.59) (end 159.5 143.59) (width 0.35) (layer B.Cu) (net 2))
 (segment (start 159.5 143.59) (end 159.43 143.52) (width 0.35) (layer B.Cu) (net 2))
 (segment (start 162.73 145.27) (end 162.73 144.54) (width 0.35) (layer F.Cu) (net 2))
 (segment (start 166.45 141.55) (end 162.73 145.27) (width 0.35) (layer F.Cu) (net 2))
 (segment (start 162.73 144.54) (end 161.78 143.59) (width 0.35) (layer F.Cu) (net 2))
 (segment (start 162.73 145.27) (end 160.67 147.33) (width 0.35) (layer F.Cu) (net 2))
 (via (at 161.78 143.59) (size 0.8) (drill 0.4) (layers F.Cu B.Cu) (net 2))
 (segment (start 160.67 147.33) (end 159.09 147.33) (width 0.35) (layer F.Cu) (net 2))
 (segment (start 159.09 147.33) (end 157.65 145.89) (width 0.35) (layer F.Cu) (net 2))
 (segment (start 157.65 145.89) (end 156.8 145.89) (width 0.35) (layer F.Cu) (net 2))
 (segment (start 166.45 141.25) (end 166.45 141.55) (width 0.35) (layer F.Cu) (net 2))
 (segment (start 171.235002 139.58) (end 168.97 139.58) (width 0.35) (layer F.Cu) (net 2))
 (segment (start 168.97 139.58) (end 167.3 141.25) (width 0.35) (layer F.Cu) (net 2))
 (segment (start 167.3 141.25) (end 166.45 141.25) (width 0.35) (layer F.Cu) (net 2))
 (segment (start 176.21 131.13) (end 176.21 134.605002) (width 0.35) (layer F.Cu) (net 2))
 (segment (start 178.03 129.01) (end 178.03 129.31) (width 0.35) (layer F.Cu) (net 2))
 (segment (start 178.03 129.31) (end 176.21 131.13) (width 0.35) (layer F.Cu) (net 2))
 (segment (start 185.84 125.03) (end 181.86 129.01) (width 0.35) (layer F.Cu) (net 2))
 (segment (start 185.84 121.83) (end 185.84 125.03) (width 0.35) (layer F.Cu) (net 2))
 (segment (start 184.33 119.17) (end 184.33 120.32) (width 0.35) (layer F.Cu) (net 2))
 (segment (start 184.33 120.32) (end 185.84 121.83) (width 0.35) (layer F.Cu) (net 2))
 (segment (start 188.15 116.93) (end 185.91 119.17) (width 0.35) (layer F.Cu) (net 2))
 (segment (start 185.91 119.17) (end 184.33 119.17) (width 0.35) (layer F.Cu) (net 2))
 (segment (start 188.15 111) (end 188.15 116.93) (width 0.35) (layer F.Cu) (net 2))
 (segment (start 186.41 108.11) (end 186.41 109.26) (width 0.35) (layer F.Cu) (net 2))
 (segment (start 188.3 100.19) (end 188.3 105.07) (width 0.35) (layer F.Cu) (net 2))
 (segment (start 188.3 105.07) (end 186.41 106.96) (width 0.35) (layer F.Cu) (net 2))
 (segment (start 186.41 106.96) (end 186.41 108.11) (width 0.35) (layer F.Cu) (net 2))
 (segment (start 186.21 97.8) (end 186.21 98.1) (width 0.35) (layer F.Cu) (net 2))
 (segment (start 186.21 98.1) (end 188.3 100.19) (width 0.35) (layer F.Cu) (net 2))
 (segment (start 182.184102 89.79) (end 182.96765 89.79) (width 0.35) (layer F.Cu) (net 2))
 (segment (start 182.96765 89.79) (end 186.21 93.03235) (width 0.35) (layer F.Cu) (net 2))
 (segment (start 186.21 93.03235) (end 186.21 96.65) (width 0.35) (layer F.Cu) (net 2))
 (segment (start 186.21 96.65) (end 186.21 97.8) (width 0.35) (layer F.Cu) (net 2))
 (segment (start 156.8 140.89) (end 156.8 141.19) (width 0.25) (layer F.Cu) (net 4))
 (segment (start 153.91 144.08) (end 151.85 144.08) (width 0.25) (layer F.Cu) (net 4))
 (segment (start 156.8 141.19) (end 153.91 144.08) (width 0.25) (layer F.Cu) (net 4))
 (segment (start 151.85 144.08) (end 150.75 144.08) (width 0.25) (layer F.Cu) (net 4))
 (segment (start 178.03 134.31) (end 171.09 141.25) (width 0.35) (layer F.Cu) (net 5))
 (segment (start 171.09 141.25) (end 170.5 141.25) (width 0.35) (layer F.Cu) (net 5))
 (segment (start 170.5 141.25) (end 169.65 141.25) (width 0.35) (layer F.Cu) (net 5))
 (segment (start 178.03 134.01) (end 178.03 134.31) (width 0.25) (layer F.Cu) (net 5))
 (segment (start 166.45 136.25) (end 166.45 137.4) (width 0.35) (layer F.Cu) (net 3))
 (segment (start 166.45 137.4) (end 160 143.85) (width 0.35) (layer F.Cu) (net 3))
 (segment (start 160 143.85) (end 160 144.74) (width 0.35) (layer F.Cu) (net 3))
 (segment (start 160 144.74) (end 160 145.89) (width 0.35) (layer F.Cu) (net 3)))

